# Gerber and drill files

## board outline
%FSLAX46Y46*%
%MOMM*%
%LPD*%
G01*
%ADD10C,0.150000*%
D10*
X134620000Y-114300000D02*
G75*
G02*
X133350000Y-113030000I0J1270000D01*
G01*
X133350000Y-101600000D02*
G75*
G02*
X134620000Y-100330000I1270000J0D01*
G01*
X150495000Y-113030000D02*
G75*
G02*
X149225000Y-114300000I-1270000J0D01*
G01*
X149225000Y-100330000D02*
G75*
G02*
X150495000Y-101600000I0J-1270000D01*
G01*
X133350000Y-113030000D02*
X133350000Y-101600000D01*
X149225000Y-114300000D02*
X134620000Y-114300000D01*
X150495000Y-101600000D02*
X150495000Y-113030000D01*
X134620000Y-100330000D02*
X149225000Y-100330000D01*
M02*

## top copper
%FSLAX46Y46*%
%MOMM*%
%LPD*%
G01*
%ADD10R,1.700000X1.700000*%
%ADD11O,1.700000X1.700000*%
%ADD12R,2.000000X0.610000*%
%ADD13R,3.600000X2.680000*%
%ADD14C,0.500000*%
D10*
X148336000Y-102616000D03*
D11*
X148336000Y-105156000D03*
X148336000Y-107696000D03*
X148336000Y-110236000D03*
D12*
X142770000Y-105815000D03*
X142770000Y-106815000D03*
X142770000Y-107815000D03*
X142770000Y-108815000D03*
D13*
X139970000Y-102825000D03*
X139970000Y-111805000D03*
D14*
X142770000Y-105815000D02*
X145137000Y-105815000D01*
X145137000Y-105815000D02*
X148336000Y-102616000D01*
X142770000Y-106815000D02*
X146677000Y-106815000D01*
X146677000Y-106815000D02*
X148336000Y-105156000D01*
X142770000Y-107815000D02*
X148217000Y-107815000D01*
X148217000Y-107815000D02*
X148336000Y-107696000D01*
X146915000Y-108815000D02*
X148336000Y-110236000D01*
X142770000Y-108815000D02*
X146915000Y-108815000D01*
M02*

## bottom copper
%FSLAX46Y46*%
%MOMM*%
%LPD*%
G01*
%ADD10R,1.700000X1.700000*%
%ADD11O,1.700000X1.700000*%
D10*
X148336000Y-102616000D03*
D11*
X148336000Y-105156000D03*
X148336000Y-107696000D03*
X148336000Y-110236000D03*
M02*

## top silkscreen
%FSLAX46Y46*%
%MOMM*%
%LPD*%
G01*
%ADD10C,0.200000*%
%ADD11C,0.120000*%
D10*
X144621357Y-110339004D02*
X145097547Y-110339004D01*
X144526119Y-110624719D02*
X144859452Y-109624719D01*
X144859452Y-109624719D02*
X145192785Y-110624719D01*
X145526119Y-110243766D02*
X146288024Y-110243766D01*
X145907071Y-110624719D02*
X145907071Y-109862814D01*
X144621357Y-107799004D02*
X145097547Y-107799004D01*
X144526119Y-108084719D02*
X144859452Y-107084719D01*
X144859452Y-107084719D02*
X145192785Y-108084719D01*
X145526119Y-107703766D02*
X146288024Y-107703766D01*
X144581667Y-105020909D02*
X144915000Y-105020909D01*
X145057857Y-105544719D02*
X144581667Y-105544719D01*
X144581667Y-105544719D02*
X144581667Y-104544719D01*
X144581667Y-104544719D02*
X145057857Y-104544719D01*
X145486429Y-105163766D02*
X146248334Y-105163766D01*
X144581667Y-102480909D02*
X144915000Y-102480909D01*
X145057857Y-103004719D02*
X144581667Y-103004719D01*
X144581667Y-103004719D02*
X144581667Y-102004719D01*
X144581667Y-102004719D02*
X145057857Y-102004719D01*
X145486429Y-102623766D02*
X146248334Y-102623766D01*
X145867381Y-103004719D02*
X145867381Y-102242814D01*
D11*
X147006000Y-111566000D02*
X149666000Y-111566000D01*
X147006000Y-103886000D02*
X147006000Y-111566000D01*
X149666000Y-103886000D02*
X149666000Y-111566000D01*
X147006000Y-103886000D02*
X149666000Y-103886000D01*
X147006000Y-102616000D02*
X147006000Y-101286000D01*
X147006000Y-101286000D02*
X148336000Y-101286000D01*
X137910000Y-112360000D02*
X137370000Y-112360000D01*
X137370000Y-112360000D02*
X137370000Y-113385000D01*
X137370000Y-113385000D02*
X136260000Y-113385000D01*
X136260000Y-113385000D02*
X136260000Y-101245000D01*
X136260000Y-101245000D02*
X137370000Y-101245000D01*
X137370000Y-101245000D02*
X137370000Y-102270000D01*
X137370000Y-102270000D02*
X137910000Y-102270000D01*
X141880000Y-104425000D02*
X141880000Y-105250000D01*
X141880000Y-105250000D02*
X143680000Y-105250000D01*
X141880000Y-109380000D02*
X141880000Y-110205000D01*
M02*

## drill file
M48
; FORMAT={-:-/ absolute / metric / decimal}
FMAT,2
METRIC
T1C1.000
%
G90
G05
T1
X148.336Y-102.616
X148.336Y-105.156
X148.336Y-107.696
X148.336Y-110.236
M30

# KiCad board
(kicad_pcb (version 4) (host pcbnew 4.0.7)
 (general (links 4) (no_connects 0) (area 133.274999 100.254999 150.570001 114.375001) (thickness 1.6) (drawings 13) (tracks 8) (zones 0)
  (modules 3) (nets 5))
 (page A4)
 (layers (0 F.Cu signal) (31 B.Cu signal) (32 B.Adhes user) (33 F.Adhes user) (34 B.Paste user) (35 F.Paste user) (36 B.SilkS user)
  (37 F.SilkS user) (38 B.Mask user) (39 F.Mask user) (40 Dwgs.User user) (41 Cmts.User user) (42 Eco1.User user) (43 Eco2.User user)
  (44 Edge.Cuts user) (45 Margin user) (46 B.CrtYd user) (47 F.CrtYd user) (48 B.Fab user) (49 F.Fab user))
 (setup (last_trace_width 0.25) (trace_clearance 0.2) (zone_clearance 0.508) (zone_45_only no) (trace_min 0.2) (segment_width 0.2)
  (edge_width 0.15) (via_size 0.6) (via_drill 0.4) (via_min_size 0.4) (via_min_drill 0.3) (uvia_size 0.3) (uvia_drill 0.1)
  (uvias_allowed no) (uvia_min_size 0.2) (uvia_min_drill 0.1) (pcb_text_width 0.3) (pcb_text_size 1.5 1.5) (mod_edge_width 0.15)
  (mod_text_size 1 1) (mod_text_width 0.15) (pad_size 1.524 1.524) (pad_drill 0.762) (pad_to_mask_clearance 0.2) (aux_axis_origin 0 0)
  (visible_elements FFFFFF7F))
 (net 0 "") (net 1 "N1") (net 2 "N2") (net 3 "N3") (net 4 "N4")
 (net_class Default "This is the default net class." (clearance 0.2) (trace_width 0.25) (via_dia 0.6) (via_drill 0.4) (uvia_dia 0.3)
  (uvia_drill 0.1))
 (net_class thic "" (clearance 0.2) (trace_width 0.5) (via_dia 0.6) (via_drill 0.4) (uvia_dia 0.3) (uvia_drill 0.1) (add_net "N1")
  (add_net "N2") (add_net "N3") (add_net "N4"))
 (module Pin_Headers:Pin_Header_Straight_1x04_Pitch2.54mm (layer F.Cu) (at 148.336 102.616)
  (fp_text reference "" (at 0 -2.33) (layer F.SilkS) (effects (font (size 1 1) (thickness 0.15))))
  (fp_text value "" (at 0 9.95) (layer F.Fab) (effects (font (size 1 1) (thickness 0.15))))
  (fp_line (start -1.33 8.95) (end 1.33 8.95) (layer F.SilkS) (width 0.12))
  (fp_line (start -1.33 1.27) (end -1.33 8.95) (layer F.SilkS) (width 0.12))
  (fp_line (start 1.33 1.27) (end 1.33 8.95) (layer F.SilkS) (width 0.12))
  (fp_line (start -1.33 1.27) (end 1.33 1.27) (layer F.SilkS) (width 0.12))
  (fp_line (start -1.33 0) (end -1.33 -1.33) (layer F.SilkS) (width 0.12))
  (fp_line (start -1.33 -1.33) (end 0 -1.33) (layer F.SilkS) (width 0.12))
  (pad 1 thru_hole rect (at 0 0) (size 1.7 1.7) (drill 1) (layers *.Cu *.Mask) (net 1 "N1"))
  (pad 2 thru_hole oval (at 0 2.54) (size 1.7 1.7) (drill 1) (layers *.Cu *.Mask) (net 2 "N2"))
  (pad 3 thru_hole oval (at 0 5.08) (size 1.7 1.7) (drill 1) (layers *.Cu *.Mask) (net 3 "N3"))
  (pad 4 thru_hole oval (at 0 7.62) (size 1.7 1.7) (drill 1) (layers *.Cu *.Mask) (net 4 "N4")))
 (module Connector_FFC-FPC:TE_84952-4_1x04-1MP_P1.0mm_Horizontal (layer F.Cu) (at 140.97 107.315 270)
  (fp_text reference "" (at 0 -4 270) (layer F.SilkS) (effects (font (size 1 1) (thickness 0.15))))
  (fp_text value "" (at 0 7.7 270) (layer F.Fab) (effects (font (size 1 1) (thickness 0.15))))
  (fp_line (start 5.045 3.06) (end 5.045 3.6) (layer F.SilkS) (width 0.12))
  (fp_line (start 5.045 3.6) (end 6.07 3.6) (layer F.SilkS) (width 0.12))
  (fp_line (start 6.07 3.6) (end 6.07 4.71) (layer F.SilkS) (width 0.12))
  (fp_line (start 6.07 4.71) (end -6.07 4.71) (layer F.SilkS) (width 0.12))
  (fp_line (start -6.07 4.71) (end -6.07 3.6) (layer F.SilkS) (width 0.12))
  (fp_line (start -6.07 3.6) (end -5.045 3.6) (layer F.SilkS) (width 0.12))
  (fp_line (start -5.045 3.6) (end -5.045 3.06) (layer F.SilkS) (width 0.12))
  (fp_line (start -2.89 -0.91) (end -2.065 -0.91) (layer F.SilkS) (width 0.12))
  (fp_line (start -2.065 -0.91) (end -2.065 -2.71) (layer F.SilkS) (width 0.12))
  (fp_line (start 2.065 -0.91) (end 2.89 -0.91) (layer F.SilkS) (width 0.12))
  (pad 1 smd rect (at -1.5 -1.8 270) (size 0.61 2) (layers F.Cu F.Paste F.Mask) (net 1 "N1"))
  (pad 2 smd rect (at -0.5 -1.8 270) (size 0.61 2) (layers F.Cu F.Paste F.Mask) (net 2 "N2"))
  (pad 3 smd rect (at 0.5 -1.8 270) (size 0.61 2) (layers F.Cu F.Paste F.Mask) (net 3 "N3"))
  (pad 4 smd rect (at 1.5 -1.8 270) (size 0.61 2) (layers F.Cu F.Paste F.Mask) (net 4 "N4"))
  (pad MP smd rect (at -4.49 1 270) (size 2.68 3.6) (layers F.Cu F.Paste F.Mask))
  (pad MP smd rect (at 4.49 1 270) (size 2.68 3.6) (layers F.Cu F.Paste F.Mask)))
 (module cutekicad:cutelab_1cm (layer B.Cu) (at 140.462 105.918 180)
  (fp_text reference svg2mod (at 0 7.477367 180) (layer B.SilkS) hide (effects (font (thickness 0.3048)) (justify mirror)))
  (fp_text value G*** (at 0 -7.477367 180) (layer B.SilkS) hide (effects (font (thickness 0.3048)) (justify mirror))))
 (gr_arc (start 134.62 113.03) (end 134.62 114.3) (angle 90) (layer Edge.Cuts) (width 0.15))
 (gr_arc (start 134.62 101.6) (end 133.35 101.6) (angle 90) (layer Edge.Cuts) (width 0.15))
 (gr_arc (start 149.225 113.03) (end 150.495 113.03) (angle 90) (layer Edge.Cuts) (width 0.15))
 (gr_arc (start 149.225 101.6) (end 149.225 100.33) (angle 90) (layer Edge.Cuts) (width 0.15))
 (gr_line (start 133.35 113.03) (end 133.35 101.6) (angle 90) (layer Edge.Cuts) (width 0.15))
 (gr_line (start 149.225 114.3) (end 134.62 114.3) (angle 90) (layer Edge.Cuts) (width 0.15))
 (gr_line (start 150.495 101.6) (end 150.495 113.03) (angle 90) (layer Edge.Cuts) (width 0.15))
 (gr_line (start 134.62 100.33) (end 149.225 100.33) (angle 90) (layer Edge.Cuts) (width 0.15))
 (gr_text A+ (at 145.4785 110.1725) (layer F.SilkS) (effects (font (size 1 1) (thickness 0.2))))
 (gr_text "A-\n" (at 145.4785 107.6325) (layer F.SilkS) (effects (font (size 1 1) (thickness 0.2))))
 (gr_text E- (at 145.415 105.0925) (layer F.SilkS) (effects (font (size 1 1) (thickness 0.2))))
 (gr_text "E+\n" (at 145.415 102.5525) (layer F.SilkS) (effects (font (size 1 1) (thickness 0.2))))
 (segment (start 142.77 105.815) (end 145.137 105.815) (width 0.5) (layer F.Cu) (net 1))
 (segment (start 145.137 105.815) (end 148.336 102.616) (width 0.5) (layer F.Cu) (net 1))
 (segment (start 142.77 106.815) (end 146.677 106.815) (width 0.5) (layer F.Cu) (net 2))
 (segment (start 146.677 106.815) (end 148.336 105.156) (width 0.5) (layer F.Cu) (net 2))
 (segment (start 142.77 107.815) (end 148.217 107.815) (width 0.5) (layer F.Cu) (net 3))
 (segment (start 148.217 107.815) (end 148.336 107.696) (width 0.5) (layer F.Cu) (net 3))
 (segment (start 146.915 108.815) (end 148.336 110.236) (width 0.5) (layer F.Cu) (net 4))
 (segment (start 142.77 108.815) (end 146.915 108.815) (width 0.5) (layer F.Cu) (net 4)))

